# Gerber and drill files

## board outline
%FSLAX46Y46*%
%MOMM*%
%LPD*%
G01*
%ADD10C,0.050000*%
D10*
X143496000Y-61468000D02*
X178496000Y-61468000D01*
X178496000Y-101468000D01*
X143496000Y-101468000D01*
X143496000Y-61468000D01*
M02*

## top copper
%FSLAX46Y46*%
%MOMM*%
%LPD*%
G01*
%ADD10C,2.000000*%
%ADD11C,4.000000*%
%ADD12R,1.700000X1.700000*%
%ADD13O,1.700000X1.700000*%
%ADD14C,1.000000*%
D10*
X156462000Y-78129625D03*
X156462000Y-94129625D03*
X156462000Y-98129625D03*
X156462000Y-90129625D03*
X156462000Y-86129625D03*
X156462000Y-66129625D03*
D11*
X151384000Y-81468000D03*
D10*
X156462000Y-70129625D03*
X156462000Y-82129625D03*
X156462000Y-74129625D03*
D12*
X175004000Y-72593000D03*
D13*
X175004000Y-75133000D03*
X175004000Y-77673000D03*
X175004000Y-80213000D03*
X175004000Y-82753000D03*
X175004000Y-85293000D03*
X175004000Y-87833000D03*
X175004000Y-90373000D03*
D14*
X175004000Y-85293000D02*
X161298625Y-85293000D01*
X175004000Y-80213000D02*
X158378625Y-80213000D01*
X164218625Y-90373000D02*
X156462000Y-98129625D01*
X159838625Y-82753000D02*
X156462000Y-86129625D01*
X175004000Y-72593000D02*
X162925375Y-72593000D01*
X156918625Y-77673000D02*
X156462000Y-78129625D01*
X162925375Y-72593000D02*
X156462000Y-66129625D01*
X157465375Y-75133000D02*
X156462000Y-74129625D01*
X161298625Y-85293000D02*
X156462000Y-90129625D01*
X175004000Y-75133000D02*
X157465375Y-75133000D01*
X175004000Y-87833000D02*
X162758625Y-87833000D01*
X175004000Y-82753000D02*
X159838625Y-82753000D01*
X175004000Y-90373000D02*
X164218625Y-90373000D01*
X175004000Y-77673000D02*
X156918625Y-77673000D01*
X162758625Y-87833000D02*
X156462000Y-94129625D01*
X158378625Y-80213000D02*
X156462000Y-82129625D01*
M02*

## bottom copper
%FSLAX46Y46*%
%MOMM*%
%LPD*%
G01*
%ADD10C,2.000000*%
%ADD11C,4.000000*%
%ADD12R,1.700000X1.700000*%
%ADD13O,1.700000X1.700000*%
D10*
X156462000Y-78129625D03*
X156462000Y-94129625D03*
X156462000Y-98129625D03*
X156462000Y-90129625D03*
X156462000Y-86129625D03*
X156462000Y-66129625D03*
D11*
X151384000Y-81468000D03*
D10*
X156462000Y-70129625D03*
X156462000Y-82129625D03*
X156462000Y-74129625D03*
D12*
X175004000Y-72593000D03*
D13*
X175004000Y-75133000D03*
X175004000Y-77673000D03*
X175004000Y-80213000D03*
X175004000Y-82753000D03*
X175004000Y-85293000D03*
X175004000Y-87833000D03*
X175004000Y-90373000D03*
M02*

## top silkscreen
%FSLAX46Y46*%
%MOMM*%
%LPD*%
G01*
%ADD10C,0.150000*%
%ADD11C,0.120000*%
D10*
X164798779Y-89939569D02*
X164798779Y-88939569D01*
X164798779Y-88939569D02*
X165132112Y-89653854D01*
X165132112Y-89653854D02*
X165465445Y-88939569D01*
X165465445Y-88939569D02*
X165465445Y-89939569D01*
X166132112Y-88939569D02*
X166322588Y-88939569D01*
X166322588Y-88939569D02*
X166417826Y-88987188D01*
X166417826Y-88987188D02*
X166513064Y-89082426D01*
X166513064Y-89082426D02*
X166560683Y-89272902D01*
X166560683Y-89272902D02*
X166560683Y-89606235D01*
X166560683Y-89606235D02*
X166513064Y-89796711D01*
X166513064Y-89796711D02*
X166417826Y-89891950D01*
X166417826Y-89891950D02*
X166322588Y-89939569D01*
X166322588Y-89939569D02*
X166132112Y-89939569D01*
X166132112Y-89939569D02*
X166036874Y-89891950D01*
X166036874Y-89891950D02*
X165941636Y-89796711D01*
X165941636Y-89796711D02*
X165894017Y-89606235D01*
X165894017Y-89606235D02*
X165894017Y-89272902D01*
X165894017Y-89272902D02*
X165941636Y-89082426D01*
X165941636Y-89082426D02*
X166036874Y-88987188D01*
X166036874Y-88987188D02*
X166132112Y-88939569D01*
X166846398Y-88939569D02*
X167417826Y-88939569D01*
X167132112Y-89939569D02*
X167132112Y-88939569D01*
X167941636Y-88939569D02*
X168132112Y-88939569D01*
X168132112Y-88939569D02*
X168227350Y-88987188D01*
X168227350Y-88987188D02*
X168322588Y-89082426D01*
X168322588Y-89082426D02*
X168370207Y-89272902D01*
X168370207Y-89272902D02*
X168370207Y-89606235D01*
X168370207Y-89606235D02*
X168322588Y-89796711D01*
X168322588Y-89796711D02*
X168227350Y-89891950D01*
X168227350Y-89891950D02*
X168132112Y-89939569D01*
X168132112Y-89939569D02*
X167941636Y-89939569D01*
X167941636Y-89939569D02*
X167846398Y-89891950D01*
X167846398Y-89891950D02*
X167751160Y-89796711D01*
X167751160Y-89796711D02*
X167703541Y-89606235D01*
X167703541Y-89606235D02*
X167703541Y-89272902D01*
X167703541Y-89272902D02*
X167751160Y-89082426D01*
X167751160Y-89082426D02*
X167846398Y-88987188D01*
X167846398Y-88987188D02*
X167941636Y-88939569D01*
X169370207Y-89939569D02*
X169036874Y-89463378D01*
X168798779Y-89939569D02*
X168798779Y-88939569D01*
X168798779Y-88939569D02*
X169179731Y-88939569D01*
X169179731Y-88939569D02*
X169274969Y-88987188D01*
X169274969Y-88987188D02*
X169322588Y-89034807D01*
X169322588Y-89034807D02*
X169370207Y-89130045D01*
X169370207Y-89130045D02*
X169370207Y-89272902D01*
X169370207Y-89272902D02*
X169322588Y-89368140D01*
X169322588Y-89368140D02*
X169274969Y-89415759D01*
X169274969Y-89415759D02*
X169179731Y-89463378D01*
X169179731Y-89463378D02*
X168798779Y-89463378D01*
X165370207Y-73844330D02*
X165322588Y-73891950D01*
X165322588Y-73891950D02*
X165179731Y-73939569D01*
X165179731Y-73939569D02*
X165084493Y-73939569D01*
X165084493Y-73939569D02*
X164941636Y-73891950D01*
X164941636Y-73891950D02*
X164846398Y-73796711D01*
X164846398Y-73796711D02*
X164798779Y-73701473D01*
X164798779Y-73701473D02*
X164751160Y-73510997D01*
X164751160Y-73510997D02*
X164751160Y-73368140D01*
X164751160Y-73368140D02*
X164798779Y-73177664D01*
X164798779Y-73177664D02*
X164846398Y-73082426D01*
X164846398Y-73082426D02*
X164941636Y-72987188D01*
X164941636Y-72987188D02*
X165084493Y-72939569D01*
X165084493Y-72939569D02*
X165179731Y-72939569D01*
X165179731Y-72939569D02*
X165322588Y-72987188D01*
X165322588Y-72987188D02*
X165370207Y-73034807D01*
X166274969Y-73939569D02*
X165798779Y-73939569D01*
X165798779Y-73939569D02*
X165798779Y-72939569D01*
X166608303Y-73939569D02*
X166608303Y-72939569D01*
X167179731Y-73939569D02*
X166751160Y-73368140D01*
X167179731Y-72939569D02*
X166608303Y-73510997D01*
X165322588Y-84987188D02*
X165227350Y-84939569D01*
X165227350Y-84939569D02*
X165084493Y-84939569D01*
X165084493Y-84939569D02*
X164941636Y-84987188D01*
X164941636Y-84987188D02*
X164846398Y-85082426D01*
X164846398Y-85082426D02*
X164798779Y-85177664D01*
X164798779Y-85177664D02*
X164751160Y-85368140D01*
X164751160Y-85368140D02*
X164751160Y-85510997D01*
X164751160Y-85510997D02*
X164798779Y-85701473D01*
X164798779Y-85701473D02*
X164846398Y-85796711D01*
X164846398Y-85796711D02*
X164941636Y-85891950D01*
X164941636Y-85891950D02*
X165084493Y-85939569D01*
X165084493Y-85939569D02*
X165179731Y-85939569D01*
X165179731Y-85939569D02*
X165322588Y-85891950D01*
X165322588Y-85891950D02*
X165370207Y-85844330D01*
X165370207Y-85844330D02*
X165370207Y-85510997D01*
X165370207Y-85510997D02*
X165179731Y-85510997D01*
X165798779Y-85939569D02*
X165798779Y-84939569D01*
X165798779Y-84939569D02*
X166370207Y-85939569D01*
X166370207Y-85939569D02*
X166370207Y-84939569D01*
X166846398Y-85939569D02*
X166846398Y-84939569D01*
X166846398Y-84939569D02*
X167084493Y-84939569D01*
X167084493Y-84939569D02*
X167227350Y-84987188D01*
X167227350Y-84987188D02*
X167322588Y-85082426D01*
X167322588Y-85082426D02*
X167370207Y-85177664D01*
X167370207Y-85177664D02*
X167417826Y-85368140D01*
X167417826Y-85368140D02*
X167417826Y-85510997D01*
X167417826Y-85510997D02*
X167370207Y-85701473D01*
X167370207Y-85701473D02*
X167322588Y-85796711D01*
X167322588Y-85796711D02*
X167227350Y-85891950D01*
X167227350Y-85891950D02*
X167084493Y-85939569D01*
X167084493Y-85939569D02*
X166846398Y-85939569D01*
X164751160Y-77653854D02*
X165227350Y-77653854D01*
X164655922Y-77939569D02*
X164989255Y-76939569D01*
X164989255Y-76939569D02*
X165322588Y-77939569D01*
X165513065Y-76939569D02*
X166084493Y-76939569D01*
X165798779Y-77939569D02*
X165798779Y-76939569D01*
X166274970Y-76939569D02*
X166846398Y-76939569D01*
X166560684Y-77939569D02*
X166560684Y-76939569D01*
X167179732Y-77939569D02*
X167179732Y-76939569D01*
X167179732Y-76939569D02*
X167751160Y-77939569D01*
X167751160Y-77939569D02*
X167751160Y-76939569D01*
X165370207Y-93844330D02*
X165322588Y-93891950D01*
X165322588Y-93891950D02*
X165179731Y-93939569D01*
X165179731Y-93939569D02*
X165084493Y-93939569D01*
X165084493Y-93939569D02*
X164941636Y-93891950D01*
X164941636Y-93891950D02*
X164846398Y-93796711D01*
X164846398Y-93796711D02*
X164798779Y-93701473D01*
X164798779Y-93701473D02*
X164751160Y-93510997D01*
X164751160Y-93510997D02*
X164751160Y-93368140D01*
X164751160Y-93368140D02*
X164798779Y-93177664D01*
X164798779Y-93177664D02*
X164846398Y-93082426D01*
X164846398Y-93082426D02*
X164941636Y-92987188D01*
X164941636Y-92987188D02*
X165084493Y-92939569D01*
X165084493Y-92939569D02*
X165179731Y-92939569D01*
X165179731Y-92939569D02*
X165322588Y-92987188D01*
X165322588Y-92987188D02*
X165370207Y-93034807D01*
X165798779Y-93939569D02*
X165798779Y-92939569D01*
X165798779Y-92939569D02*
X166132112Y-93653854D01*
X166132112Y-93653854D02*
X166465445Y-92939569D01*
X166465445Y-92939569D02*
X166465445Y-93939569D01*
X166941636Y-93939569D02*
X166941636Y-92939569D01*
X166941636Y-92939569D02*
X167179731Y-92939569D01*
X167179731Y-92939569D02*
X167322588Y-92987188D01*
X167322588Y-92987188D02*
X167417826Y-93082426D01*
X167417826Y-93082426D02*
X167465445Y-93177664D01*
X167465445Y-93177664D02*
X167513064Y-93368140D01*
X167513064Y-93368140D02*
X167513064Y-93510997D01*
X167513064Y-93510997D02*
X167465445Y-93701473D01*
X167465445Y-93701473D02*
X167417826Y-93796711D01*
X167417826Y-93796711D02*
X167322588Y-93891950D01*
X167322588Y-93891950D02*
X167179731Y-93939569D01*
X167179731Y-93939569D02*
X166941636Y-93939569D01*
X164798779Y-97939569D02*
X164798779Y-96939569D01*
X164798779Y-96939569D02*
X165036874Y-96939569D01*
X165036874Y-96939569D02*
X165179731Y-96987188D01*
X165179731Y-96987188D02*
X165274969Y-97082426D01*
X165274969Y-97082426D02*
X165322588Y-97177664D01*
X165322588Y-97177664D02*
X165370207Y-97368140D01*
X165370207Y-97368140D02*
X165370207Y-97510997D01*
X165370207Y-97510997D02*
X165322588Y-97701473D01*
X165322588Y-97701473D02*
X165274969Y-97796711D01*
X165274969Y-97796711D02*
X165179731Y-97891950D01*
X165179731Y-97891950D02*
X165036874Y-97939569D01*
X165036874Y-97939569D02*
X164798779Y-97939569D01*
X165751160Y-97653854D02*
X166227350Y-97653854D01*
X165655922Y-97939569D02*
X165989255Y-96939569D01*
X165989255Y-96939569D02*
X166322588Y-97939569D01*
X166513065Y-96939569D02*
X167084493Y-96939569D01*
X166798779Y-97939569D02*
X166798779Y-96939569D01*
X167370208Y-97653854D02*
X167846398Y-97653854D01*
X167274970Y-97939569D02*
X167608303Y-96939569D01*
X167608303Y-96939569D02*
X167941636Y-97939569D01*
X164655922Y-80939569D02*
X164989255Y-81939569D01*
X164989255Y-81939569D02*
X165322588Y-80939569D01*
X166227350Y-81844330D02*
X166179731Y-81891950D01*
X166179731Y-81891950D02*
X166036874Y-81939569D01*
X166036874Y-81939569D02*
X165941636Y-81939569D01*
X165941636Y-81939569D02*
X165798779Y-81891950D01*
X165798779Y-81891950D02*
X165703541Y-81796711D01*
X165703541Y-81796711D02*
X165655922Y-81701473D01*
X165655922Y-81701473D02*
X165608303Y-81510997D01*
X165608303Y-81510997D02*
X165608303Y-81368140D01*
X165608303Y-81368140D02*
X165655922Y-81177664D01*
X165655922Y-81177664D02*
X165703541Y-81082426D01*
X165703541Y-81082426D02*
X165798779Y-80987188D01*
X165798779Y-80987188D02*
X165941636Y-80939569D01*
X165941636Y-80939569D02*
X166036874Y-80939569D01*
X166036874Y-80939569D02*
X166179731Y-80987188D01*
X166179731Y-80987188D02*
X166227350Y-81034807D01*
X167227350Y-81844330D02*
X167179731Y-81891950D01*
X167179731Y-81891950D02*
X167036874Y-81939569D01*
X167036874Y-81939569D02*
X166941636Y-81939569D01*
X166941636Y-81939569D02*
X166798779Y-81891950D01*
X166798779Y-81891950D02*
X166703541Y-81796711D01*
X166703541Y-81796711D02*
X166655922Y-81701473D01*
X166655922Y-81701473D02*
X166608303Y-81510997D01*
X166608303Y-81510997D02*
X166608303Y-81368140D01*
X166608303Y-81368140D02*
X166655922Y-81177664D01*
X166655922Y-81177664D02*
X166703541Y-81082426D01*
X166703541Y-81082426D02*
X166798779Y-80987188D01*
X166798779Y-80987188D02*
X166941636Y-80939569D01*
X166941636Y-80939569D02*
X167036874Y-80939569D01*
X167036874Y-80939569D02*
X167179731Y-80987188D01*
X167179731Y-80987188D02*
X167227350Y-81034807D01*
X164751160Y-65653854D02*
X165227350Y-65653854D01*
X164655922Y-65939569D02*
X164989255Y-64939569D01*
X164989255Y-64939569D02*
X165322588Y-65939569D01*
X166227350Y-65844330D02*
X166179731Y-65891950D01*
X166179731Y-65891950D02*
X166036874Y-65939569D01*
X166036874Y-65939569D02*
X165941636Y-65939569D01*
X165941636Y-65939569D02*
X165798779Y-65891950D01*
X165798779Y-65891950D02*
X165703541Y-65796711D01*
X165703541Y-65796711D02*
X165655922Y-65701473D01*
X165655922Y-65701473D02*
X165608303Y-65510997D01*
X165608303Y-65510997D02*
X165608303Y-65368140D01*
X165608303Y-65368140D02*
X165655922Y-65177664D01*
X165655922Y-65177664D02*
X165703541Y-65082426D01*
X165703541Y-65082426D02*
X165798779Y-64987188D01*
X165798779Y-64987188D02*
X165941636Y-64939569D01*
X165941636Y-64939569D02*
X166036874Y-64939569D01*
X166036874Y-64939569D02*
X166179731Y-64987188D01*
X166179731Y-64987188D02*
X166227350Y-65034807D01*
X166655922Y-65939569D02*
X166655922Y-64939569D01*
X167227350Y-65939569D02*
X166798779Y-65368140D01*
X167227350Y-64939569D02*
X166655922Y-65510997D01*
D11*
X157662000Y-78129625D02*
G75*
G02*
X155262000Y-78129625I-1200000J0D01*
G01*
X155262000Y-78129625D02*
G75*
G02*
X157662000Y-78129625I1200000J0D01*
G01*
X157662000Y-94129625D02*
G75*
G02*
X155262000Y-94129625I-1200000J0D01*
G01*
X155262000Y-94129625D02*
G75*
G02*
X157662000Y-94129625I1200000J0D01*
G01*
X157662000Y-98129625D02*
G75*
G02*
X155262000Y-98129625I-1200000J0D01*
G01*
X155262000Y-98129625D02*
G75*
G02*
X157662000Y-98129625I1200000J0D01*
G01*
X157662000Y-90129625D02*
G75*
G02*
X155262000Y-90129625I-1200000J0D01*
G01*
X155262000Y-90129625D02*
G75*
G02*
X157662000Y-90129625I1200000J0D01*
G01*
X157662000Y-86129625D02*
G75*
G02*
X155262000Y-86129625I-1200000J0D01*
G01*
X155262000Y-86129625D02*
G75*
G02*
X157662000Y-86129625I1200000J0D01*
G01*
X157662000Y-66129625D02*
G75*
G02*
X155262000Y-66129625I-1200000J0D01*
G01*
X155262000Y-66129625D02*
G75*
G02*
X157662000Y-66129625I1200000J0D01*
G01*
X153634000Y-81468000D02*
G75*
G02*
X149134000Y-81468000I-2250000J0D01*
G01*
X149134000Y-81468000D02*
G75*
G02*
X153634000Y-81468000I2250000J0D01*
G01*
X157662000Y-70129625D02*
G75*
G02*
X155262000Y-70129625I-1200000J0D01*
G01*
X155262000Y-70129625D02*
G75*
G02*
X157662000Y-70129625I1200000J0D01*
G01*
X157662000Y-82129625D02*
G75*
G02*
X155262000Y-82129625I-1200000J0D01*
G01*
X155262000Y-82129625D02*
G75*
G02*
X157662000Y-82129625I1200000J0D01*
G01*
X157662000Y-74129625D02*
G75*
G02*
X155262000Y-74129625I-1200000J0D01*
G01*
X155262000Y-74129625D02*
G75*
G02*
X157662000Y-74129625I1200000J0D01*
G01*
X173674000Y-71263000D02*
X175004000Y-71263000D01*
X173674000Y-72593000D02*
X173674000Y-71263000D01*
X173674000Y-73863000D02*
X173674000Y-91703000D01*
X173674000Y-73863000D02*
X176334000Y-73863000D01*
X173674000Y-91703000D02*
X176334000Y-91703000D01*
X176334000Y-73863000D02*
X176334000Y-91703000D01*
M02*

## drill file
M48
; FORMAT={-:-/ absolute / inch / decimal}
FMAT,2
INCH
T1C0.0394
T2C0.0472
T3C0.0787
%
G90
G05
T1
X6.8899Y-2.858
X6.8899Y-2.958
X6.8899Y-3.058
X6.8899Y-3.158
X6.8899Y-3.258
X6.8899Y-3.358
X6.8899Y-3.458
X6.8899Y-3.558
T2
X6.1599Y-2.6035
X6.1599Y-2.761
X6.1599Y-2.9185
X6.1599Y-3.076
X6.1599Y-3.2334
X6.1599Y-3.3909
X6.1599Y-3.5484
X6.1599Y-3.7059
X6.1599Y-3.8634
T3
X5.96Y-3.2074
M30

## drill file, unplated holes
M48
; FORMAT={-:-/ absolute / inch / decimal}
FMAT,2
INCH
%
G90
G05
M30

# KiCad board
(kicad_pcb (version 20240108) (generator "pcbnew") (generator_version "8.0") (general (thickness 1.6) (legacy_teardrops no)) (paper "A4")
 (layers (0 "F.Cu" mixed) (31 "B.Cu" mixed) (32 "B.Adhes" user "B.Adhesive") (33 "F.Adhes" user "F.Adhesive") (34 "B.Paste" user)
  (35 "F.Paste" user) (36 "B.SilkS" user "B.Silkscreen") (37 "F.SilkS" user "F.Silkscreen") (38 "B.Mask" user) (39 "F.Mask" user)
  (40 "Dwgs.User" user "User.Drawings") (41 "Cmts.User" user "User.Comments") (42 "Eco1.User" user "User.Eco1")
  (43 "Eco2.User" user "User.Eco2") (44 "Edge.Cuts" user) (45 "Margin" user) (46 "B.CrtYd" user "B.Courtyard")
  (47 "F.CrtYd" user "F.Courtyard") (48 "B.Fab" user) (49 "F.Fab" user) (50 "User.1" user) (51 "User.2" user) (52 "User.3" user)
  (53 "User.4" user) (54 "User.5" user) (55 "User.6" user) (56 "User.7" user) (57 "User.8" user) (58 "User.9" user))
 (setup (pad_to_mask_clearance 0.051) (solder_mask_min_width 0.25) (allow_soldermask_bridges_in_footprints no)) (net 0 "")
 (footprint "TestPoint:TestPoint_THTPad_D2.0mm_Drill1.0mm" (layer "F.Cu") (at 156.462 78.129625)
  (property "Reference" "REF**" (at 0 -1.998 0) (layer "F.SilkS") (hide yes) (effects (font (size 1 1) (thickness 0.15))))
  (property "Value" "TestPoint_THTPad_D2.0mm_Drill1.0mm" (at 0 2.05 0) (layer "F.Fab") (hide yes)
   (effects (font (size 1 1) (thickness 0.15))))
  (fp_circle (center 0 0) (end 0 1.2) (stroke (width 0.12) (type solid)) (fill none) (layer "F.SilkS"))
  (pad "6" thru_hole circle (at 0 0) (size 2 2) (drill 1.2) (layers "*.Cu" "*.Mask") (remove_unused_layers no)))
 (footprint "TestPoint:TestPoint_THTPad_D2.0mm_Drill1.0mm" (layer "F.Cu") (at 156.462 94.129625)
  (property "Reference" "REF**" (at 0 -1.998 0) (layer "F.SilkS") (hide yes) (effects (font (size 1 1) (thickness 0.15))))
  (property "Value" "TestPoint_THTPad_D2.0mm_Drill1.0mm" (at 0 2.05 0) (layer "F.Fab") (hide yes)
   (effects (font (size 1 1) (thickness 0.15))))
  (fp_circle (center 0 0) (end 0 1.2) (stroke (width 0.12) (type solid)) (fill none) (layer "F.SilkS"))
  (pad "2" thru_hole circle (at 0 0) (size 2 2) (drill 1.2) (layers "*.Cu" "*.Mask") (remove_unused_layers no)))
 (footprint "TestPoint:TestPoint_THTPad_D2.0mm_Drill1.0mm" (layer "F.Cu") (at 156.462 98.129625)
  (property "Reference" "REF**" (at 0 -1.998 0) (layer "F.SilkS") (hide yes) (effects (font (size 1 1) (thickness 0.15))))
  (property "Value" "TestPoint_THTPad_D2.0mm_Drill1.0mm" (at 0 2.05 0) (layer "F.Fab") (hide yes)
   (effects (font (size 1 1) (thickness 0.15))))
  (fp_circle (center 0 0) (end 0 1.2) (stroke (width 0.12) (type solid)) (fill none) (layer "F.SilkS"))
  (pad "1" thru_hole circle (at 0 0) (size 2 2) (drill 1.2) (layers "*.Cu" "*.Mask") (remove_unused_layers no)))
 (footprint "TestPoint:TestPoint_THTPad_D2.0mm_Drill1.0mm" (layer "F.Cu") (at 156.462 90.129625)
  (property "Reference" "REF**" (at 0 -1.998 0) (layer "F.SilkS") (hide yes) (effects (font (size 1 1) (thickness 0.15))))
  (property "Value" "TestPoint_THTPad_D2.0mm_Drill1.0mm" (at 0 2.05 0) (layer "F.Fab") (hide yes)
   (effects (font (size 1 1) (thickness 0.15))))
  (fp_circle (center 0 0) (end 0 1.2) (stroke (width 0.12) (type solid)) (fill none) (layer "F.SilkS"))
  (pad "3" thru_hole circle (at 0 0) (size 2 2) (drill 1.2) (layers "*.Cu" "*.Mask") (remove_unused_layers no)))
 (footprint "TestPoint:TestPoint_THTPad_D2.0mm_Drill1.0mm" (layer "F.Cu") (at 156.462 86.129625)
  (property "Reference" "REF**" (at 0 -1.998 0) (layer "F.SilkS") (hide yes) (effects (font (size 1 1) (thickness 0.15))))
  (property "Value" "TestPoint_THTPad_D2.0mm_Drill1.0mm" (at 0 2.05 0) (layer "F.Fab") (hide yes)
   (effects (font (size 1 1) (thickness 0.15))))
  (fp_circle (center 0 0) (end 0 1.2) (stroke (width 0.12) (type solid)) (fill none) (layer "F.SilkS"))
  (pad "4" thru_hole circle (at 0 0) (size 2 2) (drill 1.2) (layers "*.Cu" "*.Mask") (remove_unused_layers no)))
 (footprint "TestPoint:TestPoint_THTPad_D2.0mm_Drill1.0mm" (layer "F.Cu") (at 156.462 66.129625)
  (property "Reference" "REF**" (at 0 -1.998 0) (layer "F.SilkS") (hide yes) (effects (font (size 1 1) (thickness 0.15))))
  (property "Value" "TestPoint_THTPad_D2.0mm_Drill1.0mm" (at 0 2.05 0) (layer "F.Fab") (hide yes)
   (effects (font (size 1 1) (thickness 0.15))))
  (fp_circle (center 0 0) (end 0 1.2) (stroke (width 0.12) (type solid)) (fill none) (layer "F.SilkS"))
  (pad "9" thru_hole circle (at 0 0) (size 2 2) (drill 1.2) (layers "*.Cu" "*.Mask") (remove_unused_layers no)))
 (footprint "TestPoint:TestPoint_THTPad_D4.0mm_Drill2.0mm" (layer "F.Cu") (at 151.384 81.468)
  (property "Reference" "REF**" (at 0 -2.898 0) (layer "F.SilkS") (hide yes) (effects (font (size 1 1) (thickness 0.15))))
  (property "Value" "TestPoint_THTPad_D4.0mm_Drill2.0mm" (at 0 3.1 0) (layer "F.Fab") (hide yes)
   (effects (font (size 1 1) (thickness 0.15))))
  (fp_circle (center 0 0) (end 0 2.25) (stroke (width 0.12) (type solid)) (fill none) (layer "F.SilkS"))
  (pad "1" thru_hole circle (at 0 0) (size 4 4) (drill 2) (layers "*.Cu" "*.Mask") (remove_unused_layers no)))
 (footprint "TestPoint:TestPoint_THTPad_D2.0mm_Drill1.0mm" (layer "F.Cu") (at 156.462 70.129625)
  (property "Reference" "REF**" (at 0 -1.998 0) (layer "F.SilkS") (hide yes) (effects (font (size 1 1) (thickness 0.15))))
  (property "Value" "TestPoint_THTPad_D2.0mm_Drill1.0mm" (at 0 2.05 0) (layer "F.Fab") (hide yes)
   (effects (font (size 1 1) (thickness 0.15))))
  (fp_circle (center 0 0) (end 0 1.2) (stroke (width 0.12) (type solid)) (fill none) (layer "F.SilkS"))
  (pad "8" thru_hole circle (at 0 0) (size 2 2) (drill 1.2) (layers "*.Cu" "*.Mask") (remove_unused_layers no)))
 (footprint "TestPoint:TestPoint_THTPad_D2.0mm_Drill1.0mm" (layer "F.Cu") (at 156.462 82.129625)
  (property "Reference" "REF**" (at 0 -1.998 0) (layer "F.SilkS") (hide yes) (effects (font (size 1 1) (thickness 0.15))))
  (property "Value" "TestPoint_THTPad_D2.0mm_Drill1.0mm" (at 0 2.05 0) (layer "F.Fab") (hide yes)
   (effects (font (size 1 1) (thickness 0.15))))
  (fp_circle (center 0 0) (end 0 1.2) (stroke (width 0.12) (type solid)) (fill none) (layer "F.SilkS"))
  (pad "5" thru_hole circle (at 0 0) (size 2 2) (drill 1.2) (layers "*.Cu" "*.Mask") (remove_unused_layers no)))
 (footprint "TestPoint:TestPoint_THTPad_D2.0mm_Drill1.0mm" (layer "F.Cu") (at 156.462 74.129625)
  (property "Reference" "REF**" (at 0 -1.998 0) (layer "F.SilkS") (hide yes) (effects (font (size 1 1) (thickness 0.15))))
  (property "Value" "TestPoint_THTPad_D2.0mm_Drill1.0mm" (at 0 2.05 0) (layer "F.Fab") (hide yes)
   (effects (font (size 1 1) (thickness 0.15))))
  (fp_circle (center 0 0) (end 0 1.2) (stroke (width 0.12) (type solid)) (fill none) (layer "F.SilkS"))
  (pad "7" thru_hole circle (at 0 0) (size 2 2) (drill 1.2) (layers "*.Cu" "*.Mask") (remove_unused_layers no)))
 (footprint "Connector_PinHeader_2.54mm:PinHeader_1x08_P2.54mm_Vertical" (layer "F.Cu") (at 175.004 72.593)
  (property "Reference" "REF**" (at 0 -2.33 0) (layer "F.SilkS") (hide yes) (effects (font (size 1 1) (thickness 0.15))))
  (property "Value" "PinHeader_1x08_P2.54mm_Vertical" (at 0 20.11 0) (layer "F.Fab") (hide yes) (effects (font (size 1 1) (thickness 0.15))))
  (fp_line (start -1.33 -1.33) (end 0 -1.33) (stroke (width 0.12) (type solid)) (layer "F.SilkS"))
  (fp_line (start -1.33 0) (end -1.33 -1.33) (stroke (width 0.12) (type solid)) (layer "F.SilkS"))
  (fp_line (start -1.33 1.27) (end -1.33 19.11) (stroke (width 0.12) (type solid)) (layer "F.SilkS"))
  (fp_line (start -1.33 1.27) (end 1.33 1.27) (stroke (width 0.12) (type solid)) (layer "F.SilkS"))
  (fp_line (start -1.33 19.11) (end 1.33 19.11) (stroke (width 0.12) (type solid)) (layer "F.SilkS"))
  (fp_line (start 1.33 1.27) (end 1.33 19.11) (stroke (width 0.12) (type solid)) (layer "F.SilkS"))
  (pad "1" thru_hole rect (at 0 0) (size 1.7 1.7) (drill 1) (layers "*.Cu" "*.Mask") (remove_unused_layers no))
  (pad "2" thru_hole oval (at 0 2.54) (size 1.7 1.7) (drill 1) (layers "*.Cu" "*.Mask") (remove_unused_layers no))
  (pad "3" thru_hole oval (at 0 5.08) (size 1.7 1.7) (drill 1) (layers "*.Cu" "*.Mask") (remove_unused_layers no))
  (pad "4" thru_hole oval (at 0 7.62) (size 1.7 1.7) (drill 1) (layers "*.Cu" "*.Mask") (remove_unused_layers no))
  (pad "5" thru_hole oval (at 0 10.16) (size 1.7 1.7) (drill 1) (layers "*.Cu" "*.Mask") (remove_unused_layers no))
  (pad "6" thru_hole oval (at 0 12.7) (size 1.7 1.7) (drill 1) (layers "*.Cu" "*.Mask") (remove_unused_layers no))
  (pad "7" thru_hole oval (at 0 15.24) (size 1.7 1.7) (drill 1) (layers "*.Cu" "*.Mask") (remove_unused_layers no))
  (pad "8" thru_hole oval (at 0 17.78) (size 1.7 1.7) (drill 1) (layers "*.Cu" "*.Mask") (remove_unused_layers no)))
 (gr_rect (start 143.496 61.468) (end 178.496 101.468) (stroke (width 0.05) (type default)) (fill none) (layer "Edge.Cuts"))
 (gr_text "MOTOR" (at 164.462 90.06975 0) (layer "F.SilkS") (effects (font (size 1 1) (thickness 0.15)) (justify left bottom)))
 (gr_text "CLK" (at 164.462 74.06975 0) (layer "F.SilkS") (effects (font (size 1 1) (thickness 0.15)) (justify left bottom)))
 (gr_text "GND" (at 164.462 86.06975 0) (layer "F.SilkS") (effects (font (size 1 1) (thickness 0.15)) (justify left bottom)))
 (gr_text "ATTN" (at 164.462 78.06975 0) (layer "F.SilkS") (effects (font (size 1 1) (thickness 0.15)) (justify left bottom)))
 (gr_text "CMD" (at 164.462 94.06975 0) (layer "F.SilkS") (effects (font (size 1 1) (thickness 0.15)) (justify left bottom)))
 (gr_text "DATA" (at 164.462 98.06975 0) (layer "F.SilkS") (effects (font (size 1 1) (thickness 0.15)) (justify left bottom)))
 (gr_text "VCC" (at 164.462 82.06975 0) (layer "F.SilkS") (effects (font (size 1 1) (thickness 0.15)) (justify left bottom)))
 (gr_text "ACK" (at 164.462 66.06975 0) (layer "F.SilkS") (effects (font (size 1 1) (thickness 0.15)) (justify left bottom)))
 (segment (start 175.004 85.293) (end 161.298625 85.293) (width 1) (layer "F.Cu") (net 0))
 (segment (start 175.004 80.213) (end 158.378625 80.213) (width 1) (layer "F.Cu") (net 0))
 (segment (start 164.218625 90.373) (end 156.462 98.129625) (width 1) (layer "F.Cu") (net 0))
 (segment (start 159.838625 82.753) (end 156.462 86.129625) (width 1) (layer "F.Cu") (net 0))
 (segment (start 175.004 72.593) (end 162.925375 72.593) (width 1) (layer "F.Cu") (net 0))
 (segment (start 156.918625 77.673) (end 156.462 78.129625) (width 1) (layer "F.Cu") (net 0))
 (segment (start 162.925375 72.593) (end 156.462 66.129625) (width 1) (layer "F.Cu") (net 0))
 (segment (start 157.465375 75.133) (end 156.462 74.129625) (width 1) (layer "F.Cu") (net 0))
 (segment (start 161.298625 85.293) (end 156.462 90.129625) (width 1) (layer "F.Cu") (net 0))
 (segment (start 175.004 75.133) (end 157.465375 75.133) (width 1) (layer "F.Cu") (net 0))
 (segment (start 175.004 87.833) (end 162.758625 87.833) (width 1) (layer "F.Cu") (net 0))
 (segment (start 175.004 82.753) (end 159.838625 82.753) (width 1) (layer "F.Cu") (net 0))
 (segment (start 175.004 90.373) (end 164.218625 90.373) (width 1) (layer "F.Cu") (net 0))
 (segment (start 175.004 77.673) (end 156.918625 77.673) (width 1) (layer "F.Cu") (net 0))
 (segment (start 162.758625 87.833) (end 156.462 94.129625) (width 1) (layer "F.Cu") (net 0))
 (segment (start 158.378625 80.213) (end 156.462 82.129625) (width 1) (layer "F.Cu") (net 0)))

